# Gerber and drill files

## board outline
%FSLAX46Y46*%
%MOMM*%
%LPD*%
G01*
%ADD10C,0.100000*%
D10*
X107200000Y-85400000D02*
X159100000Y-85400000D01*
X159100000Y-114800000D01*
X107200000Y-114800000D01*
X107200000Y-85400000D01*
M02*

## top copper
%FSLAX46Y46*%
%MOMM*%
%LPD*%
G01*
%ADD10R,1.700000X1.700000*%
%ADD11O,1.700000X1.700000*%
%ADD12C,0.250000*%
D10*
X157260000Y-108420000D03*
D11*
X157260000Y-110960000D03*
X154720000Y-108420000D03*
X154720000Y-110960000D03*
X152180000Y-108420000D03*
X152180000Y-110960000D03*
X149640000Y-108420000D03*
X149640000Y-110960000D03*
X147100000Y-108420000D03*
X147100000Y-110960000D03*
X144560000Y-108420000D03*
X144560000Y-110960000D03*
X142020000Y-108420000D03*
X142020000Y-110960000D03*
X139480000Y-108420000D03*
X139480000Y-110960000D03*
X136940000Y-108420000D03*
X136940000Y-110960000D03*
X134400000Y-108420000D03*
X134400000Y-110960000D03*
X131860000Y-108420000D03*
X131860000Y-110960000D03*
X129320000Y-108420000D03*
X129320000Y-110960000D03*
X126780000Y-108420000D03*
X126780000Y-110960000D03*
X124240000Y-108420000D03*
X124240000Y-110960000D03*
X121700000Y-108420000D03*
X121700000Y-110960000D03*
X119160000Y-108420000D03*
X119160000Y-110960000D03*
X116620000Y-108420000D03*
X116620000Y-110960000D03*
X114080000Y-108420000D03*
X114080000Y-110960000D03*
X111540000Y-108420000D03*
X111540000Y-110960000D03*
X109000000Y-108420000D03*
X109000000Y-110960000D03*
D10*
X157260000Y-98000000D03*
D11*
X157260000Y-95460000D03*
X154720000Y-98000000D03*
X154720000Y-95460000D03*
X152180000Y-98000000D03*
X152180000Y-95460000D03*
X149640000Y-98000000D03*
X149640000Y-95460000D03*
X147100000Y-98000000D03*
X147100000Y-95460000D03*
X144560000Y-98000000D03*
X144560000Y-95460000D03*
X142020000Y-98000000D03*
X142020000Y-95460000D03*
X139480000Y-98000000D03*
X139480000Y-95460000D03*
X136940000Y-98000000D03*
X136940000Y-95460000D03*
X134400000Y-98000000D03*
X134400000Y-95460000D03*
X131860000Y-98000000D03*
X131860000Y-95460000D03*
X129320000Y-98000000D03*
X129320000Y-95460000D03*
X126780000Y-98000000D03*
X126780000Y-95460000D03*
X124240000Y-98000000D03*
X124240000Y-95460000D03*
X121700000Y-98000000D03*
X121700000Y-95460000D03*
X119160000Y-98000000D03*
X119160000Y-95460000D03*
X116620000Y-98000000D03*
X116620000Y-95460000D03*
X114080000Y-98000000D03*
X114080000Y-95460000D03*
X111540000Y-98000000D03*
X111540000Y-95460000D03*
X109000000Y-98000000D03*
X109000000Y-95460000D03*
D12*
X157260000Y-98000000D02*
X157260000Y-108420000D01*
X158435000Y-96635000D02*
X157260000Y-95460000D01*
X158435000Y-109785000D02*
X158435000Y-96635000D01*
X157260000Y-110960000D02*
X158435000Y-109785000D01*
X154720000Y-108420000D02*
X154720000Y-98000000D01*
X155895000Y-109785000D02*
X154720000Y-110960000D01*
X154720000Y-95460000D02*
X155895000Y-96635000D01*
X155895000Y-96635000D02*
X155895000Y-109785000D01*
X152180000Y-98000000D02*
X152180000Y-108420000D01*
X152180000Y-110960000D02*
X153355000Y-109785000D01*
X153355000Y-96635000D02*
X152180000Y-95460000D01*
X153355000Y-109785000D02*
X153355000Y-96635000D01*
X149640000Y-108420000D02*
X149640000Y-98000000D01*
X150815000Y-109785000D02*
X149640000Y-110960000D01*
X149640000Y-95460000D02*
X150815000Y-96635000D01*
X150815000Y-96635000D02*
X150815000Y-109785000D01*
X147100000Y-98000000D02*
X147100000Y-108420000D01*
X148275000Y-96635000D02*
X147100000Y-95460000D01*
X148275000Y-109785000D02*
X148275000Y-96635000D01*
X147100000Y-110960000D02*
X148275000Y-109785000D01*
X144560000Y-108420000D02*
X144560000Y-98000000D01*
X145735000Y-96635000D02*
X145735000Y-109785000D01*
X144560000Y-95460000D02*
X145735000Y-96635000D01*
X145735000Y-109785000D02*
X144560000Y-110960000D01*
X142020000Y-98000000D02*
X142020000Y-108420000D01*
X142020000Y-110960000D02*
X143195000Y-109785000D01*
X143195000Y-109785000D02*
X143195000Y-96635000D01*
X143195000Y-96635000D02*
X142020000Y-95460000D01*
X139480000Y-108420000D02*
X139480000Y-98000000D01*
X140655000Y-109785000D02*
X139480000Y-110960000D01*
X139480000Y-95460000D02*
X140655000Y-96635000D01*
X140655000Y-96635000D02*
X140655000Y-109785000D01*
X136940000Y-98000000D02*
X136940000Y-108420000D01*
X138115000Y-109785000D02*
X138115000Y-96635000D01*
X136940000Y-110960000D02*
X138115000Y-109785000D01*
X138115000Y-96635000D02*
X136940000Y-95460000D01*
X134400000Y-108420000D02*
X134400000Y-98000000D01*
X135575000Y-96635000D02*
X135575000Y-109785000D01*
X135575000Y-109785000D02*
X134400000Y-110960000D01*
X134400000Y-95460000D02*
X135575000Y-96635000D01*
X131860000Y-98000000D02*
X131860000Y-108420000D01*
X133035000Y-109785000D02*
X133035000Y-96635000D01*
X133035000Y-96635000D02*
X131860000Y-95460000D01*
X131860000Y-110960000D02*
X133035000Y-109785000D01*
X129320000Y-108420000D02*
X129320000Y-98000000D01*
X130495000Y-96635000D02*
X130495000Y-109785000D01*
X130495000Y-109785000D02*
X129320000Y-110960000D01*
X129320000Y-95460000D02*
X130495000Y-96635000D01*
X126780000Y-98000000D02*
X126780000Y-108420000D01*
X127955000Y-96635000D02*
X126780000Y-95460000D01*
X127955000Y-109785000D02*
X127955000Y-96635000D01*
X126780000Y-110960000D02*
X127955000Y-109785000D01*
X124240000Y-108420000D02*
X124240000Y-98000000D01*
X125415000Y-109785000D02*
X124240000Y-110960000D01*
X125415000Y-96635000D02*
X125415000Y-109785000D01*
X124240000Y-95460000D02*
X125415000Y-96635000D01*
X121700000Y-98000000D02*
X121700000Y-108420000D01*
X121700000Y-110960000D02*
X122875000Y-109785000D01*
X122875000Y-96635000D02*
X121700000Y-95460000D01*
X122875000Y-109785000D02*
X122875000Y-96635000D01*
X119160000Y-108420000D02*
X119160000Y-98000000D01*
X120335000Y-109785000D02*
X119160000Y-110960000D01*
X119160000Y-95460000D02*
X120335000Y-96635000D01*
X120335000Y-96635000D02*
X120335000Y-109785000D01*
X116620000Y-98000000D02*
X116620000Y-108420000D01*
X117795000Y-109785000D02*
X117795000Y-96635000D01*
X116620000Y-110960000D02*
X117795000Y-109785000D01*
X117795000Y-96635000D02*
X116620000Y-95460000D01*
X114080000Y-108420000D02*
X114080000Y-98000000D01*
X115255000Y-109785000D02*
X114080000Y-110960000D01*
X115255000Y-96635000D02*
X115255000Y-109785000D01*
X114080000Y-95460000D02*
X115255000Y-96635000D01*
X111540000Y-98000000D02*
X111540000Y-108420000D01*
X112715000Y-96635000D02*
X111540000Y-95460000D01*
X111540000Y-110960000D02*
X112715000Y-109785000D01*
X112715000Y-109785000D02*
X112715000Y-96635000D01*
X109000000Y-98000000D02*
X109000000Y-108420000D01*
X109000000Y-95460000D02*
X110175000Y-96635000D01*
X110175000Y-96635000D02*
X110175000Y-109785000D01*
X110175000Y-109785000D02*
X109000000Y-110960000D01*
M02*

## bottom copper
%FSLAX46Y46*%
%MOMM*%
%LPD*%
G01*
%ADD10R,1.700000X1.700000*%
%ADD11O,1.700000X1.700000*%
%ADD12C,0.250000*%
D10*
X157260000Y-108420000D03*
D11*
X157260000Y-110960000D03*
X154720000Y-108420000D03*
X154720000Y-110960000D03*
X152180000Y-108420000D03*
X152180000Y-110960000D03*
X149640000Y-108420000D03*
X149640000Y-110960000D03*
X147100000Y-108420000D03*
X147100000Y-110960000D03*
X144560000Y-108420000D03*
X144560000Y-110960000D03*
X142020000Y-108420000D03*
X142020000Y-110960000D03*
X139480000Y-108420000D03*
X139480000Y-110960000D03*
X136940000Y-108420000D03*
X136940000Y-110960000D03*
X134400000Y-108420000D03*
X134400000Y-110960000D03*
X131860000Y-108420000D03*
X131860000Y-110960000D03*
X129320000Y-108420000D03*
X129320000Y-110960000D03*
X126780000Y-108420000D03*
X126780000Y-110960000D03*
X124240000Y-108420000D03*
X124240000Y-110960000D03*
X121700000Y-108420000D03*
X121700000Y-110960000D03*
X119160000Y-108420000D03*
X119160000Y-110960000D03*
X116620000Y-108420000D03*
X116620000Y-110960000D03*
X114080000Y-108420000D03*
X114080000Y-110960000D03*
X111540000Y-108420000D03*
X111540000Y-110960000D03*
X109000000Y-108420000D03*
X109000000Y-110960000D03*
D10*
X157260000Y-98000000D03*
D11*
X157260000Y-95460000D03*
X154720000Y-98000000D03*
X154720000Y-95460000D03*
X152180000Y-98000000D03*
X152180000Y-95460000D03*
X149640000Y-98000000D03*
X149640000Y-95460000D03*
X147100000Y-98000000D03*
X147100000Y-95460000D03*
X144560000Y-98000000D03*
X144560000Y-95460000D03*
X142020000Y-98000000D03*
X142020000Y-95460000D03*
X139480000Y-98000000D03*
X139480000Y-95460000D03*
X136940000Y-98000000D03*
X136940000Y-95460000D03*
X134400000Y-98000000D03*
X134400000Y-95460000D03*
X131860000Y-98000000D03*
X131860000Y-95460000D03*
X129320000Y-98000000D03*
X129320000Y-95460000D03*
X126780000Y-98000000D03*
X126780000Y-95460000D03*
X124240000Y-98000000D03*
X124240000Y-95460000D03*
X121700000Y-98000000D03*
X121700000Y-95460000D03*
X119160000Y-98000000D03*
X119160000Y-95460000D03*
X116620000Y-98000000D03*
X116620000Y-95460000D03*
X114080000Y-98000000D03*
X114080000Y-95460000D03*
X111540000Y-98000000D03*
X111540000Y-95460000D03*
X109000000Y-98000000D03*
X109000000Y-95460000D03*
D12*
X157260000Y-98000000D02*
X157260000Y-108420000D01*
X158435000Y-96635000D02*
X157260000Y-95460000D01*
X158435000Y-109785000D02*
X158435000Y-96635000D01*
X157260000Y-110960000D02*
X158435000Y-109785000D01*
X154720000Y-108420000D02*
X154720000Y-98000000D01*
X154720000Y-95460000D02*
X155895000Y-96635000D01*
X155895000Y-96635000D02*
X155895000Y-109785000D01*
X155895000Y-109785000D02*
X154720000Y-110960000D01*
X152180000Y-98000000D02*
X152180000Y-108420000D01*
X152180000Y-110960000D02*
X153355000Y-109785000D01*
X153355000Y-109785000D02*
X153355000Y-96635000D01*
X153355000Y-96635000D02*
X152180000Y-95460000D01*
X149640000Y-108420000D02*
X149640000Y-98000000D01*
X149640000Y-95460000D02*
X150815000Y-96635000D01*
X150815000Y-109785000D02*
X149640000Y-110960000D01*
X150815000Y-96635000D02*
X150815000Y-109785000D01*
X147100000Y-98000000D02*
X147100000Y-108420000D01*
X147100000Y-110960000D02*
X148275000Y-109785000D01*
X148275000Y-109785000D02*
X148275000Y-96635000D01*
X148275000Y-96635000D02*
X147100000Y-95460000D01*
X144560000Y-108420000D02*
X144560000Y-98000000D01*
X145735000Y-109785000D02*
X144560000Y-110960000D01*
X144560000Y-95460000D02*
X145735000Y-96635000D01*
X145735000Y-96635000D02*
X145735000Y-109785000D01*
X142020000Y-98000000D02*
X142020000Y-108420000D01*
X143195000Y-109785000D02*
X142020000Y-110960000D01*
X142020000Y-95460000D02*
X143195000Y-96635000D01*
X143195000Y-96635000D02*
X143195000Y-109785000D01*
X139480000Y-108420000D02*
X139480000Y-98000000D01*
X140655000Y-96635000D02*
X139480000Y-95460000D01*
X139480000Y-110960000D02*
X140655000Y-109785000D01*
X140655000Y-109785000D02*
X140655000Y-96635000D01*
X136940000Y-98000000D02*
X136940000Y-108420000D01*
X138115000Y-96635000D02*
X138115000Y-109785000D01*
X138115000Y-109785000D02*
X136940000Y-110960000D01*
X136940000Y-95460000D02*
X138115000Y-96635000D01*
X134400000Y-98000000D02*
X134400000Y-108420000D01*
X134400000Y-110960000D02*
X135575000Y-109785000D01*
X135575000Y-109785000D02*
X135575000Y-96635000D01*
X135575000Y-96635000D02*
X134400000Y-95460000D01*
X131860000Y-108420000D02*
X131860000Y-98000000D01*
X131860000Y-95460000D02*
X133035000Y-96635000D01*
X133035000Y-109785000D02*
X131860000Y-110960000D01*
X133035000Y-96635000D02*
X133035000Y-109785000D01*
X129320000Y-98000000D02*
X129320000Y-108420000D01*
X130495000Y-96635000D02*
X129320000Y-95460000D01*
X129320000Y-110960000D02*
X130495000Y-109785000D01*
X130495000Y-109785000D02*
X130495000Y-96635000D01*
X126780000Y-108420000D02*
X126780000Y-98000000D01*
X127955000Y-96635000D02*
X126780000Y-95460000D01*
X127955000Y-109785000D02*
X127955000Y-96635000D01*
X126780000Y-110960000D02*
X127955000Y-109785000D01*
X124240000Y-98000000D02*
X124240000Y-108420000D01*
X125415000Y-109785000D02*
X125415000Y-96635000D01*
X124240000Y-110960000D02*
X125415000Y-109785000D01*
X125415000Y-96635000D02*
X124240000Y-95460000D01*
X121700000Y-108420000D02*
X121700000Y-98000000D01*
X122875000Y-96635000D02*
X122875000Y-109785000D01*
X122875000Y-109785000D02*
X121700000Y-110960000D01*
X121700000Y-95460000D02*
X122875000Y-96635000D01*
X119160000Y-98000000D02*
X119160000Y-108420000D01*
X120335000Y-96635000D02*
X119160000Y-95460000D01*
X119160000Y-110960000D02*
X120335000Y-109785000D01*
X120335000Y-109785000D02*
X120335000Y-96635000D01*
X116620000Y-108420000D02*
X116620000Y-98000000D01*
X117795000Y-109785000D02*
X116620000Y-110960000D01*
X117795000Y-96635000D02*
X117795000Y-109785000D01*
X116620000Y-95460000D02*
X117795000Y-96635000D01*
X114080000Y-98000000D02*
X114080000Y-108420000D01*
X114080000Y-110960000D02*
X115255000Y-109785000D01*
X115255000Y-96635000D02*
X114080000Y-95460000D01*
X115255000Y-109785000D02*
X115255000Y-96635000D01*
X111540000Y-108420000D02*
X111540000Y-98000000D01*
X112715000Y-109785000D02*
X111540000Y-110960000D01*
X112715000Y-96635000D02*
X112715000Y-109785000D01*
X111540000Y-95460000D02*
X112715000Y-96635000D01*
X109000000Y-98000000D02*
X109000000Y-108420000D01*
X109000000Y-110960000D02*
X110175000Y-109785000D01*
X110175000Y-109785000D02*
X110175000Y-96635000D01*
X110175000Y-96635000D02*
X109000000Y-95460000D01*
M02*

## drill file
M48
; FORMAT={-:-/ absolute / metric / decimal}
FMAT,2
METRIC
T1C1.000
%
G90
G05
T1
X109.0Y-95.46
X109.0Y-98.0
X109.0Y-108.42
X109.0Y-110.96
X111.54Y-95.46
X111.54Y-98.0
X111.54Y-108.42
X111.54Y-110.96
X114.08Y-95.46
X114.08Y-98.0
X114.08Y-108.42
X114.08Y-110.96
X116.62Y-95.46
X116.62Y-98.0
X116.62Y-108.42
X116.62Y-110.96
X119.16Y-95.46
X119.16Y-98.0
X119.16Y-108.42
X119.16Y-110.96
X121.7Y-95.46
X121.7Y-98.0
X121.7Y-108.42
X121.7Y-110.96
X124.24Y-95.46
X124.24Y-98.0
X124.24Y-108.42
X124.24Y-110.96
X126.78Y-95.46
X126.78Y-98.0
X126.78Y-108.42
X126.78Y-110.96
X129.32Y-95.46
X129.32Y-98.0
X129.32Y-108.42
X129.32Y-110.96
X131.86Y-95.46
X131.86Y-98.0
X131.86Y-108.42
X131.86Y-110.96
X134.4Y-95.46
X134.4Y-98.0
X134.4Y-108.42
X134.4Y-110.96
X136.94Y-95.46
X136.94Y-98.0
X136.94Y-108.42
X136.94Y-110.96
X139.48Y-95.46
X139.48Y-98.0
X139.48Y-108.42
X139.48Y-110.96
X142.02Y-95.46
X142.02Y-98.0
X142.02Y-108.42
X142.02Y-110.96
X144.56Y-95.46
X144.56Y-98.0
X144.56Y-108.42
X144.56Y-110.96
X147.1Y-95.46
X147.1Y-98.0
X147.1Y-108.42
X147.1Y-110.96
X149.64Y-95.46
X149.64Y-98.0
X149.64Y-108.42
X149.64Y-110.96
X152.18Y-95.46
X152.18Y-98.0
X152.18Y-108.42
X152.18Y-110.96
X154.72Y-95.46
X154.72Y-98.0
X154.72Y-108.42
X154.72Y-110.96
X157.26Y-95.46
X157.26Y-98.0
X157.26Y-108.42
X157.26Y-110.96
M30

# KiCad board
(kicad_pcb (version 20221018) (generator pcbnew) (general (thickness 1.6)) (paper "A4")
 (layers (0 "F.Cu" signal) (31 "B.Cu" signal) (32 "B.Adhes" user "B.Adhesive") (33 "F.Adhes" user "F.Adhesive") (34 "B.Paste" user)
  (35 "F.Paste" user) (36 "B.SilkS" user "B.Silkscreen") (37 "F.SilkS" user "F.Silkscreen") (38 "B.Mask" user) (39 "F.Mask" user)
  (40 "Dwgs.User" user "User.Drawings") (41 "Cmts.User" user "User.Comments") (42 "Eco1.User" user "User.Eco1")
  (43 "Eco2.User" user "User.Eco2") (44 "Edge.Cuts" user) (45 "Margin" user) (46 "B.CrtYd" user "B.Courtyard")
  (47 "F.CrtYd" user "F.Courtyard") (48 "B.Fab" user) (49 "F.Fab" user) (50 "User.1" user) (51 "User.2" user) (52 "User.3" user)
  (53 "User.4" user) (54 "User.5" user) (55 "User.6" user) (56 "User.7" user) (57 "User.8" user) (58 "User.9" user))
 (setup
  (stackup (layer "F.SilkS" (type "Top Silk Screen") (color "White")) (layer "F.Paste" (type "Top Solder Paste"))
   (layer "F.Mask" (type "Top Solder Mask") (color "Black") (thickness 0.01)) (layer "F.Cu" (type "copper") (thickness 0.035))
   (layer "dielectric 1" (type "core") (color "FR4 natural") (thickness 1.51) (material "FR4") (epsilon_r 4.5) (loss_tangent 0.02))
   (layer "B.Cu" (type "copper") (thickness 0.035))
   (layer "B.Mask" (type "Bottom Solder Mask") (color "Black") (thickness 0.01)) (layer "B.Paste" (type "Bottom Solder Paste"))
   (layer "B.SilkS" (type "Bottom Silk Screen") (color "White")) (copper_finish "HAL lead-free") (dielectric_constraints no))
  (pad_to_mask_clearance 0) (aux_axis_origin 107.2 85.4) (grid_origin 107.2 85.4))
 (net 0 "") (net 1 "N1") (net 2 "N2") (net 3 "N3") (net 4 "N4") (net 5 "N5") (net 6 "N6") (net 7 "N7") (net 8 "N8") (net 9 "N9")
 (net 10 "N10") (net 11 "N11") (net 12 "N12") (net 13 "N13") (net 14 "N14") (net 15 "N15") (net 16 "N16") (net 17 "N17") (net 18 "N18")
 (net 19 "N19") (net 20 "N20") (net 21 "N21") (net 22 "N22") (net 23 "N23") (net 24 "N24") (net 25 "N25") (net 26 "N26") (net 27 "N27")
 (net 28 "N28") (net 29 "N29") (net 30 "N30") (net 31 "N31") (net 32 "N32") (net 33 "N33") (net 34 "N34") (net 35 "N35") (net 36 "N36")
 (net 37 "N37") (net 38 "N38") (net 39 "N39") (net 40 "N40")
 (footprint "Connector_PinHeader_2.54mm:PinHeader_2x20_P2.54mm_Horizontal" (layer "F.Cu") (at 157.26 108.42 -90)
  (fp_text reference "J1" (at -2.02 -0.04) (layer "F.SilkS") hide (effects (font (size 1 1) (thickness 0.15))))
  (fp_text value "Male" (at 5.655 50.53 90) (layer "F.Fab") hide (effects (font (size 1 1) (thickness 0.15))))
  (pad "1" thru_hole rect (at 0 0 270) (size 1.7 1.7) (drill 1) (layers "*.Cu" "*.Mask") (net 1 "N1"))
  (pad "2" thru_hole oval (at 2.54 0 270) (size 1.7 1.7) (drill 1) (layers "*.Cu" "*.Mask") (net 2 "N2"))
  (pad "3" thru_hole oval (at 0 2.54 270) (size 1.7 1.7) (drill 1) (layers "*.Cu" "*.Mask") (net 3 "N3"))
  (pad "4" thru_hole oval (at 2.54 2.54 270) (size 1.7 1.7) (drill 1) (layers "*.Cu" "*.Mask") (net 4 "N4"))
  (pad "5" thru_hole oval (at 0 5.08 270) (size 1.7 1.7) (drill 1) (layers "*.Cu" "*.Mask") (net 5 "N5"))
  (pad "6" thru_hole oval (at 2.54 5.08 270) (size 1.7 1.7) (drill 1) (layers "*.Cu" "*.Mask") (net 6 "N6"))
  (pad "7" thru_hole oval (at 0 7.62 270) (size 1.7 1.7) (drill 1) (layers "*.Cu" "*.Mask") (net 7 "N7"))
  (pad "8" thru_hole oval (at 2.54 7.62 270) (size 1.7 1.7) (drill 1) (layers "*.Cu" "*.Mask") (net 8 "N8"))
  (pad "9" thru_hole oval (at 0 10.16 270) (size 1.7 1.7) (drill 1) (layers "*.Cu" "*.Mask") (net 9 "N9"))
  (pad "10" thru_hole oval (at 2.54 10.16 270) (size 1.7 1.7) (drill 1) (layers "*.Cu" "*.Mask") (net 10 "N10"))
  (pad "11" thru_hole oval (at 0 12.7 270) (size 1.7 1.7) (drill 1) (layers "*.Cu" "*.Mask") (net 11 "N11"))
  (pad "12" thru_hole oval (at 2.54 12.7 270) (size 1.7 1.7) (drill 1) (layers "*.Cu" "*.Mask") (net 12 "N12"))
  (pad "13" thru_hole oval (at 0 15.24 270) (size 1.7 1.7) (drill 1) (layers "*.Cu" "*.Mask") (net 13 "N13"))
  (pad "14" thru_hole oval (at 2.54 15.24 270) (size 1.7 1.7) (drill 1) (layers "*.Cu" "*.Mask") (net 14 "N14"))
  (pad "15" thru_hole oval (at 0 17.78 270) (size 1.7 1.7) (drill 1) (layers "*.Cu" "*.Mask") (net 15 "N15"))
  (pad "16" thru_hole oval (at 2.54 17.78 270) (size 1.7 1.7) (drill 1) (layers "*.Cu" "*.Mask") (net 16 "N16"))
  (pad "17" thru_hole oval (at 0 20.32 270) (size 1.7 1.7) (drill 1) (layers "*.Cu" "*.Mask") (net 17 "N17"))
  (pad "18" thru_hole oval (at 2.54 20.32 270) (size 1.7 1.7) (drill 1) (layers "*.Cu" "*.Mask") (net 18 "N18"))
  (pad "19" thru_hole oval (at 0 22.86 270) (size 1.7 1.7) (drill 1) (layers "*.Cu" "*.Mask") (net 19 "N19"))
  (pad "20" thru_hole oval (at 2.54 22.86 270) (size 1.7 1.7) (drill 1) (layers "*.Cu" "*.Mask") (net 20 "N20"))
  (pad "21" thru_hole oval (at 0 25.4 270) (size 1.7 1.7) (drill 1) (layers "*.Cu" "*.Mask") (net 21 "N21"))
  (pad "22" thru_hole oval (at 2.54 25.4 270) (size 1.7 1.7) (drill 1) (layers "*.Cu" "*.Mask") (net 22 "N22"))
  (pad "23" thru_hole oval (at 0 27.94 270) (size 1.7 1.7) (drill 1) (layers "*.Cu" "*.Mask") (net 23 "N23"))
  (pad "24" thru_hole oval (at 2.54 27.94 270) (size 1.7 1.7) (drill 1) (layers "*.Cu" "*.Mask") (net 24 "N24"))
  (pad "25" thru_hole oval (at 0 30.48 270) (size 1.7 1.7) (drill 1) (layers "*.Cu" "*.Mask") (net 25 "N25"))
  (pad "26" thru_hole oval (at 2.54 30.48 270) (size 1.7 1.7) (drill 1) (layers "*.Cu" "*.Mask") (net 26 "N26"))
  (pad "27" thru_hole oval (at 0 33.02 270) (size 1.7 1.7) (drill 1) (layers "*.Cu" "*.Mask") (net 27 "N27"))
  (pad "28" thru_hole oval (at 2.54 33.02 270) (size 1.7 1.7) (drill 1) (layers "*.Cu" "*.Mask") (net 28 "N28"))
  (pad "29" thru_hole oval (at 0 35.56 270) (size 1.7 1.7) (drill 1) (layers "*.Cu" "*.Mask") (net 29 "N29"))
  (pad "30" thru_hole oval (at 2.54 35.56 270) (size 1.7 1.7) (drill 1) (layers "*.Cu" "*.Mask") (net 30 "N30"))
  (pad "31" thru_hole oval (at 0 38.1 270) (size 1.7 1.7) (drill 1) (layers "*.Cu" "*.Mask") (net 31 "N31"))
  (pad "32" thru_hole oval (at 2.54 38.1 270) (size 1.7 1.7) (drill 1) (layers "*.Cu" "*.Mask") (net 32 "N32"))
  (pad "33" thru_hole oval (at 0 40.64 270) (size 1.7 1.7) (drill 1) (layers "*.Cu" "*.Mask") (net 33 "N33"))
  (pad "34" thru_hole oval (at 2.54 40.64 270) (size 1.7 1.7) (drill 1) (layers "*.Cu" "*.Mask") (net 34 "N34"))
  (pad "35" thru_hole oval (at 0 43.18 270) (size 1.7 1.7) (drill 1) (layers "*.Cu" "*.Mask") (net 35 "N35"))
  (pad "36" thru_hole oval (at 2.54 43.18 270) (size 1.7 1.7) (drill 1) (layers "*.Cu" "*.Mask") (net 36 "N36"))
  (pad "37" thru_hole oval (at 0 45.72 270) (size 1.7 1.7) (drill 1) (layers "*.Cu" "*.Mask") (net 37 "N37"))
  (pad "38" thru_hole oval (at 2.54 45.72 270) (size 1.7 1.7) (drill 1) (layers "*.Cu" "*.Mask") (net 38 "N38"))
  (pad "39" thru_hole oval (at 0 48.26 270) (size 1.7 1.7) (drill 1) (layers "*.Cu" "*.Mask") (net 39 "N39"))
  (pad "40" thru_hole oval (at 2.54 48.26 270) (size 1.7 1.7) (drill 1) (layers "*.Cu" "*.Mask") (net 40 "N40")))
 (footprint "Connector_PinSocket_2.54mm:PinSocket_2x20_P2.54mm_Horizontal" (layer "F.Cu") (at 157.26 98 -90)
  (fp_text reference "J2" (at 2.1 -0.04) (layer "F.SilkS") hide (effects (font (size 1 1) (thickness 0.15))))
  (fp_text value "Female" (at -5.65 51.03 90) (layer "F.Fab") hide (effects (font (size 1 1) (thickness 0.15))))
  (pad "1" thru_hole rect (at 0 0 270) (size 1.7 1.7) (drill 1) (layers "*.Cu" "*.Mask") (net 1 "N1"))
  (pad "2" thru_hole oval (at -2.54 0 270) (size 1.7 1.7) (drill 1) (layers "*.Cu" "*.Mask") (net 2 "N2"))
  (pad "3" thru_hole oval (at 0 2.54 270) (size 1.7 1.7) (drill 1) (layers "*.Cu" "*.Mask") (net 3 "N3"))
  (pad "4" thru_hole oval (at -2.54 2.54 270) (size 1.7 1.7) (drill 1) (layers "*.Cu" "*.Mask") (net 4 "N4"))
  (pad "5" thru_hole oval (at 0 5.08 270) (size 1.7 1.7) (drill 1) (layers "*.Cu" "*.Mask") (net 5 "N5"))
  (pad "6" thru_hole oval (at -2.54 5.08 270) (size 1.7 1.7) (drill 1) (layers "*.Cu" "*.Mask") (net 6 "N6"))
  (pad "7" thru_hole oval (at 0 7.62 270) (size 1.7 1.7) (drill 1) (layers "*.Cu" "*.Mask") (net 7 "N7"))
  (pad "8" thru_hole oval (at -2.54 7.62 270) (size 1.7 1.7) (drill 1) (layers "*.Cu" "*.Mask") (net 8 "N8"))
  (pad "9" thru_hole oval (at 0 10.16 270) (size 1.7 1.7) (drill 1) (layers "*.Cu" "*.Mask") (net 9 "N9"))
  (pad "10" thru_hole oval (at -2.54 10.16 270) (size 1.7 1.7) (drill 1) (layers "*.Cu" "*.Mask") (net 10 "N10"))
  (pad "11" thru_hole oval (at 0 12.7 270) (size 1.7 1.7) (drill 1) (layers "*.Cu" "*.Mask") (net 11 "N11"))
  (pad "12" thru_hole oval (at -2.54 12.7 270) (size 1.7 1.7) (drill 1) (layers "*.Cu" "*.Mask") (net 12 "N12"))
  (pad "13" thru_hole oval (at 0 15.24 270) (size 1.7 1.7) (drill 1) (layers "*.Cu" "*.Mask") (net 13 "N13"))
  (pad "14" thru_hole oval (at -2.54 15.24 270) (size 1.7 1.7) (drill 1) (layers "*.Cu" "*.Mask") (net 14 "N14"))
  (pad "15" thru_hole oval (at 0 17.78 270) (size 1.7 1.7) (drill 1) (layers "*.Cu" "*.Mask") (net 15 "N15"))
  (pad "16" thru_hole oval (at -2.54 17.78 270) (size 1.7 1.7) (drill 1) (layers "*.Cu" "*.Mask") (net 16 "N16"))
  (pad "17" thru_hole oval (at 0 20.32 270) (size 1.7 1.7) (drill 1) (layers "*.Cu" "*.Mask") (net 17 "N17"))
  (pad "18" thru_hole oval (at -2.54 20.32 270) (size 1.7 1.7) (drill 1) (layers "*.Cu" "*.Mask") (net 18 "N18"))
  (pad "19" thru_hole oval (at 0 22.86 270) (size 1.7 1.7) (drill 1) (layers "*.Cu" "*.Mask") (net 19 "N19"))
  (pad "20" thru_hole oval (at -2.54 22.86 270) (size 1.7 1.7) (drill 1) (layers "*.Cu" "*.Mask") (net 20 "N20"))
  (pad "21" thru_hole oval (at 0 25.4 270) (size 1.7 1.7) (drill 1) (layers "*.Cu" "*.Mask") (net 21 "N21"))
  (pad "22" thru_hole oval (at -2.54 25.4 270) (size 1.7 1.7) (drill 1) (layers "*.Cu" "*.Mask") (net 22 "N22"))
  (pad "23" thru_hole oval (at 0 27.94 270) (size 1.7 1.7) (drill 1) (layers "*.Cu" "*.Mask") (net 23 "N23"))
  (pad "24" thru_hole oval (at -2.54 27.94 270) (size 1.7 1.7) (drill 1) (layers "*.Cu" "*.Mask") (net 24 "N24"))
  (pad "25" thru_hole oval (at 0 30.48 270) (size 1.7 1.7) (drill 1) (layers "*.Cu" "*.Mask") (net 25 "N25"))
  (pad "26" thru_hole oval (at -2.54 30.48 270) (size 1.7 1.7) (drill 1) (layers "*.Cu" "*.Mask") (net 26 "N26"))
  (pad "27" thru_hole oval (at 0 33.02 270) (size 1.7 1.7) (drill 1) (layers "*.Cu" "*.Mask") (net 27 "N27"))
  (pad "28" thru_hole oval (at -2.54 33.02 270) (size 1.7 1.7) (drill 1) (layers "*.Cu" "*.Mask") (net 28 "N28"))
  (pad "29" thru_hole oval (at 0 35.56 270) (size 1.7 1.7) (drill 1) (layers "*.Cu" "*.Mask") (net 29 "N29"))
  (pad "30" thru_hole oval (at -2.54 35.56 270) (size 1.7 1.7) (drill 1) (layers "*.Cu" "*.Mask") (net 30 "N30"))
  (pad "31" thru_hole oval (at 0 38.1 270) (size 1.7 1.7) (drill 1) (layers "*.Cu" "*.Mask") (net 31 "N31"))
  (pad "32" thru_hole oval (at -2.54 38.1 270) (size 1.7 1.7) (drill 1) (layers "*.Cu" "*.Mask") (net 32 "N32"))
  (pad "33" thru_hole oval (at 0 40.64 270) (size 1.7 1.7) (drill 1) (layers "*.Cu" "*.Mask") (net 33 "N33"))
  (pad "34" thru_hole oval (at -2.54 40.64 270) (size 1.7 1.7) (drill 1) (layers "*.Cu" "*.Mask") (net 34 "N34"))
  (pad "35" thru_hole oval (at 0 43.18 270) (size 1.7 1.7) (drill 1) (layers "*.Cu" "*.Mask") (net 35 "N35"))
  (pad "36" thru_hole oval (at -2.54 43.18 270) (size 1.7 1.7) (drill 1) (layers "*.Cu" "*.Mask") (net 36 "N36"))
  (pad "37" thru_hole oval (at 0 45.72 270) (size 1.7 1.7) (drill 1) (layers "*.Cu" "*.Mask") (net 37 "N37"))
  (pad "38" thru_hole oval (at -2.54 45.72 270) (size 1.7 1.7) (drill 1) (layers "*.Cu" "*.Mask") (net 38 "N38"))
  (pad "39" thru_hole oval (at 0 48.26 270) (size 1.7 1.7) (drill 1) (layers "*.Cu" "*.Mask") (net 39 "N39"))
  (pad "40" thru_hole oval (at -2.54 48.26 270) (size 1.7 1.7) (drill 1) (layers "*.Cu" "*.Mask") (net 40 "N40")))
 (gr_rect (start 107.2 85.4) (end 159.1 114.8) (stroke (width 0.1) (type default)) (fill none) (layer "Edge.Cuts"))
 (segment (start 157.26 98) (end 157.26 108.42) (width 0.25) (layer "F.Cu") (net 1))
 (segment (start 157.26 98) (end 157.26 108.42) (width 0.25) (layer "B.Cu") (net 1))
 (segment (start 158.435 96.635) (end 157.26 95.46) (width 0.25) (layer "F.Cu") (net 2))
 (segment (start 158.435 109.785) (end 158.435 96.635) (width 0.25) (layer "F.Cu") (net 2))
 (segment (start 157.26 110.96) (end 158.435 109.785) (width 0.25) (layer "F.Cu") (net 2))
 (segment (start 158.435 96.635) (end 157.26 95.46) (width 0.25) (layer "B.Cu") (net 2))
 (segment (start 158.435 109.785) (end 158.435 96.635) (width 0.25) (layer "B.Cu") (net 2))
 (segment (start 157.26 110.96) (end 158.435 109.785) (width 0.25) (layer "B.Cu") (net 2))
 (segment (start 154.72 108.42) (end 154.72 98) (width 0.25) (layer "F.Cu") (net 3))
 (segment (start 154.72 108.42) (end 154.72 98) (width 0.25) (layer "B.Cu") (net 3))
 (segment (start 155.895 109.785) (end 154.72 110.96) (width 0.25) (layer "F.Cu") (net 4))
 (segment (start 154.72 95.46) (end 155.895 96.635) (width 0.25) (layer "F.Cu") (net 4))
 (segment (start 155.895 96.635) (end 155.895 109.785) (width 0.25) (layer "F.Cu") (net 4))
 (segment (start 154.72 95.46) (end 155.895 96.635) (width 0.25) (layer "B.Cu") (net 4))
 (segment (start 155.895 96.635) (end 155.895 109.785) (width 0.25) (layer "B.Cu") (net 4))
 (segment (start 155.895 109.785) (end 154.72 110.96) (width 0.25) (layer "B.Cu") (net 4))
 (segment (start 152.18 98) (end 152.18 108.42) (width 0.25) (layer "F.Cu") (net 5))
 (segment (start 152.18 98) (end 152.18 108.42) (width 0.25) (layer "B.Cu") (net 5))
 (segment (start 152.18 110.96) (end 153.355 109.785) (width 0.25) (layer "F.Cu") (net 6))
 (segment (start 153.355 96.635) (end 152.18 95.46) (width 0.25) (layer "F.Cu") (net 6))
 (segment (start 153.355 109.785) (end 153.355 96.635) (width 0.25) (layer "F.Cu") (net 6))
 (segment (start 152.18 110.96) (end 153.355 109.785) (width 0.25) (layer "B.Cu") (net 6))
 (segment (start 153.355 109.785) (end 153.355 96.635) (width 0.25) (layer "B.Cu") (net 6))
 (segment (start 153.355 96.635) (end 152.18 95.46) (width 0.25) (layer "B.Cu") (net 6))
 (segment (start 149.64 108.42) (end 149.64 98) (width 0.25) (layer "F.Cu") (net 7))
 (segment (start 149.64 108.42) (end 149.64 98) (width 0.25) (layer "B.Cu") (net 7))
 (segment (start 150.815 109.785) (end 149.64 110.96) (width 0.25) (layer "F.Cu") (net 8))
 (segment (start 149.64 95.46) (end 150.815 96.635) (width 0.25) (layer "F.Cu") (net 8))
 (segment (start 150.815 96.635) (end 150.815 109.785) (width 0.25) (layer "F.Cu") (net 8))
 (segment (start 149.64 95.46) (end 150.815 96.635) (width 0.25) (layer "B.Cu") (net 8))
 (segment (start 150.815 109.785) (end 149.64 110.96) (width 0.25) (layer "B.Cu") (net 8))
 (segment (start 150.815 96.635) (end 150.815 109.785) (width 0.25) (layer "B.Cu") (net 8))
 (segment (start 147.1 98) (end 147.1 108.42) (width 0.25) (layer "F.Cu") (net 9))
 (segment (start 147.1 98) (end 147.1 108.42) (width 0.25) (layer "B.Cu") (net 9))
 (segment (start 148.275 96.635) (end 147.1 95.46) (width 0.25) (layer "F.Cu") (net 10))
 (segment (start 148.275 109.785) (end 148.275 96.635) (width 0.25) (layer "F.Cu") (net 10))
 (segment (start 147.1 110.96) (end 148.275 109.785) (width 0.25) (layer "F.Cu") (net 10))
 (segment (start 147.1 110.96) (end 148.275 109.785) (width 0.25) (layer "B.Cu") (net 10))
 (segment (start 148.275 109.785) (end 148.275 96.635) (width 0.25) (layer "B.Cu") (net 10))
 (segment (start 148.275 96.635) (end 147.1 95.46) (width 0.25) (layer "B.Cu") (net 10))
 (segment (start 144.56 108.42) (end 144.56 98) (width 0.25) (layer "F.Cu") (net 11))
 (segment (start 144.56 108.42) (end 144.56 98) (width 0.25) (layer "B.Cu") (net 11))
 (segment (start 145.735 96.635) (end 145.735 109.785) (width 0.25) (layer "F.Cu") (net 12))
 (segment (start 144.56 95.46) (end 145.735 96.635) (width 0.25) (layer "F.Cu") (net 12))
 (segment (start 145.735 109.785) (end 144.56 110.96) (width 0.25) (layer "F.Cu") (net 12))
 (segment (start 145.735 109.785) (end 144.56 110.96) (width 0.25) (layer "B.Cu") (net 12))
 (segment (start 144.56 95.46) (end 145.735 96.635) (width 0.25) (layer "B.Cu") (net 12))
 (segment (start 145.735 96.635) (end 145.735 109.785) (width 0.25) (layer "B.Cu") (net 12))
 (segment (start 142.02 98) (end 142.02 108.42) (width 0.25) (layer "F.Cu") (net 13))
 (segment (start 142.02 98) (end 142.02 108.42) (width 0.25) (layer "B.Cu") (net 13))
 (segment (start 142.02 110.96) (end 143.195 109.785) (width 0.25) (layer "F.Cu") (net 14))
 (segment (start 143.195 109.785) (end 143.195 96.635) (width 0.25) (layer "F.Cu") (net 14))
 (segment (start 143.195 96.635) (end 142.02 95.46) (width 0.25) (layer "F.Cu") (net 14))
 (segment (start 143.195 109.785) (end 142.02 110.96) (width 0.25) (layer "B.Cu") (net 14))
 (segment (start 142.02 95.46) (end 143.195 96.635) (width 0.25) (layer "B.Cu") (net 14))
 (segment (start 143.195 96.635) (end 143.195 109.785) (width 0.25) (layer "B.Cu") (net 14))
 (segment (start 139.48 108.42) (end 139.48 98) (width 0.25) (layer "F.Cu") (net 15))
 (segment (start 139.48 108.42) (end 139.48 98) (width 0.25) (layer "B.Cu") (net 15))
 (segment (start 140.655 109.785) (end 139.48 110.96) (width 0.25) (layer "F.Cu") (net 16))
 (segment (start 139.48 95.46) (end 140.655 96.635) (width 0.25) (layer "F.Cu") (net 16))
 (segment (start 140.655 96.635) (end 140.655 109.785) (width 0.25) (layer "F.Cu") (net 16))
 (segment (start 140.655 96.635) (end 139.48 95.46) (width 0.25) (layer "B.Cu") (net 16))
 (segment (start 139.48 110.96) (end 140.655 109.785) (width 0.25) (layer "B.Cu") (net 16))
 (segment (start 140.655 109.785) (end 140.655 96.635) (width 0.25) (layer "B.Cu") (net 16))
 (segment (start 136.94 98) (end 136.94 108.42) (width 0.25) (layer "F.Cu") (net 17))
 (segment (start 136.94 98) (end 136.94 108.42) (width 0.25) (layer "B.Cu") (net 17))
 (segment (start 138.115 109.785) (end 138.115 96.635) (width 0.25) (layer "F.Cu") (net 18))
 (segment (start 136.94 110.96) (end 138.115 109.785) (width 0.25) (layer "F.Cu") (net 18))
 (segment (start 138.115 96.635) (end 136.94 95.46) (width 0.25) (layer "F.Cu") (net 18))
 (segment (start 138.115 96.635) (end 138.115 109.785) (width 0.25) (layer "B.Cu") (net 18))
 (segment (start 138.115 109.785) (end 136.94 110.96) (width 0.25) (layer "B.Cu") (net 18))
 (segment (start 136.94 95.46) (end 138.115 96.635) (width 0.25) (layer "B.Cu") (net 18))
 (segment (start 134.4 108.42) (end 134.4 98) (width 0.25) (layer "F.Cu") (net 19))
 (segment (start 134.4 98) (end 134.4 108.42) (width 0.25) (layer "B.Cu") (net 19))
 (segment (start 135.575 96.635) (end 135.575 109.785) (width 0.25) (layer "F.Cu") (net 20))
 (segment (start 135.575 109.785) (end 134.4 110.96) (width 0.25) (layer "F.Cu") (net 20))
 (segment (start 134.4 95.46) (end 135.575 96.635) (width 0.25) (layer "F.Cu") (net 20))
 (segment (start 134.4 110.96) (end 135.575 109.785) (width 0.25) (layer "B.Cu") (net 20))
 (segment (start 135.575 109.785) (end 135.575 96.635) (width 0.25) (layer "B.Cu") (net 20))
 (segment (start 135.575 96.635) (end 134.4 95.46) (width 0.25) (layer "B.Cu") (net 20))
 (segment (start 131.86 98) (end 131.86 108.42) (width 0.25) (layer "F.Cu") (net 21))
 (segment (start 131.86 108.42) (end 131.86 98) (width 0.25) (layer "B.Cu") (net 21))
 (segment (start 133.035 109.785) (end 133.035 96.635) (width 0.25) (layer "F.Cu") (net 22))
 (segment (start 133.035 96.635) (end 131.86 95.46) (width 0.25) (layer "F.Cu") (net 22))
 (segment (start 131.86 110.96) (end 133.035 109.785) (width 0.25) (layer "F.Cu") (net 22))
 (segment (start 131.86 95.46) (end 133.035 96.635) (width 0.25) (layer "B.Cu") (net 22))
 (segment (start 133.035 109.785) (end 131.86 110.96) (width 0.25) (layer "B.Cu") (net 22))
 (segment (start 133.035 96.635) (end 133.035 109.785) (width 0.25) (layer "B.Cu") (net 22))
 (segment (start 129.32 108.42) (end 129.32 98) (width 0.25) (layer "F.Cu") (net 23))
 (segment (start 129.32 98) (end 129.32 108.42) (width 0.25) (layer "B.Cu") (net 23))
 (segment (start 130.495 96.635) (end 130.495 109.785) (width 0.25) (layer "F.Cu") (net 24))
 (segment (start 130.495 109.785) (end 129.32 110.96) (width 0.25) (layer "F.Cu") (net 24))
 (segment (start 129.32 95.46) (end 130.495 96.635) (width 0.25) (layer "F.Cu") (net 24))
 (segment (start 130.495 96.635) (end 129.32 95.46) (width 0.25) (layer "B.Cu") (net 24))
 (segment (start 129.32 110.96) (end 130.495 109.785) (width 0.25) (layer "B.Cu") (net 24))
 (segment (start 130.495 109.785) (end 130.495 96.635) (width 0.25) (layer "B.Cu") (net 24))
 (segment (start 126.78 98) (end 126.78 108.42) (width 0.25) (layer "F.Cu") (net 25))
 (segment (start 126.78 108.42) (end 126.78 98) (width 0.25) (layer "B.Cu") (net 25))
 (segment (start 127.955 96.635) (end 126.78 95.46) (width 0.25) (layer "F.Cu") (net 26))
 (segment (start 127.955 109.785) (end 127.955 96.635) (width 0.25) (layer "F.Cu") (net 26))
 (segment (start 126.78 110.96) (end 127.955 109.785) (width 0.25) (layer "F.Cu") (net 26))
 (segment (start 127.955 96.635) (end 126.78 95.46) (width 0.25) (layer "B.Cu") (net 26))
 (segment (start 127.955 109.785) (end 127.955 96.635) (width 0.25) (layer "B.Cu") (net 26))
 (segment (start 126.78 110.96) (end 127.955 109.785) (width 0.25) (layer "B.Cu") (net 26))
 (segment (start 124.24 108.42) (end 124.24 98) (width 0.25) (layer "F.Cu") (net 27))
 (segment (start 124.24 98) (end 124.24 108.42) (width 0.25) (layer "B.Cu") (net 27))
 (segment (start 125.415 109.785) (end 124.24 110.96) (width 0.25) (layer "F.Cu") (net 28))
 (segment (start 125.415 96.635) (end 125.415 109.785) (width 0.25) (layer "F.Cu") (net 28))
 (segment (start 124.24 95.46) (end 125.415 96.635) (width 0.25) (layer "F.Cu") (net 28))
 (segment (start 125.415 109.785) (end 125.415 96.635) (width 0.25) (layer "B.Cu") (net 28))
 (segment (start 124.24 110.96) (end 125.415 109.785) (width 0.25) (layer "B.Cu") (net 28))
 (segment (start 125.415 96.635) (end 124.24 95.46) (width 0.25) (layer "B.Cu") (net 28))
 (segment (start 121.7 98) (end 121.7 108.42) (width 0.25) (layer "F.Cu") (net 29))
 (segment (start 121.7 108.42) (end 121.7 98) (width 0.25) (layer "B.Cu") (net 29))
 (segment (start 121.7 110.96) (end 122.875 109.785) (width 0.25) (layer "F.Cu") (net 30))
 (segment (start 122.875 96.635) (end 121.7 95.46) (width 0.25) (layer "F.Cu") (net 30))
 (segment (start 122.875 109.785) (end 122.875 96.635) (width 0.25) (layer "F.Cu") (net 30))
 (segment (start 122.875 96.635) (end 122.875 109.785) (width 0.25) (layer "B.Cu") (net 30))
 (segment (start 122.875 109.785) (end 121.7 110.96) (width 0.25) (layer "B.Cu") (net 30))
 (segment (start 121.7 95.46) (end 122.875 96.635) (width 0.25) (layer "B.Cu") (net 30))
 (segment (start 119.16 108.42) (end 119.16 98) (width 0.25) (layer "F.Cu") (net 31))
 (segment (start 119.16 98) (end 119.16 108.42) (width 0.25) (layer "B.Cu") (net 31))
 (segment (start 120.335 109.785) (end 119.16 110.96) (width 0.25) (layer "F.Cu") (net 32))
 (segment (start 119.16 95.46) (end 120.335 96.635) (width 0.25) (layer "F.Cu") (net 32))
 (segment (start 120.335 96.635) (end 120.335 109.785) (width 0.25) (layer "F.Cu") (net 32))
 (segment (start 120.335 96.635) (end 119.16 95.46) (width 0.25) (layer "B.Cu") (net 32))
 (segment (start 119.16 110.96) (end 120.335 109.785) (width 0.25) (layer "B.Cu") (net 32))
 (segment (start 120.335 109.785) (end 120.335 96.635) (width 0.25) (layer "B.Cu") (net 32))
 (segment (start 116.62 98) (end 116.62 108.42) (width 0.25) (layer "F.Cu") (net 33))
 (segment (start 116.62 108.42) (end 116.62 98) (width 0.25) (layer "B.Cu") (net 33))
 (segment (start 117.795 109.785) (end 117.795 96.635) (width 0.25) (layer "F.Cu") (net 34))
 (segment (start 116.62 110.96) (end 117.795 109.785) (width 0.25) (layer "F.Cu") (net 34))
 (segment (start 117.795 96.635) (end 116.62 95.46) (width 0.25) (layer "F.Cu") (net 34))
 (segment (start 117.795 109.785) (end 116.62 110.96) (width 0.25) (layer "B.Cu") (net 34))
 (segment (start 117.795 96.635) (end 117.795 109.785) (width 0.25) (layer "B.Cu") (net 34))
 (segment (start 116.62 95.46) (end 117.795 96.635) (width 0.25) (layer "B.Cu") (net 34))
 (segment (start 114.08 108.42) (end 114.08 98) (width 0.25) (layer "F.Cu") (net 35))
 (segment (start 114.08 98) (end 114.08 108.42) (width 0.25) (layer "B.Cu") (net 35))
 (segment (start 115.255 109.785) (end 114.08 110.96) (width 0.25) (layer "F.Cu") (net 36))
 (segment (start 115.255 96.635) (end 115.255 109.785) (width 0.25) (layer "F.Cu") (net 36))
 (segment (start 114.08 95.46) (end 115.255 96.635) (width 0.25) (layer "F.Cu") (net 36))
 (segment (start 114.08 110.96) (end 115.255 109.785) (width 0.25) (layer "B.Cu") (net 36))
 (segment (start 115.255 96.635) (end 114.08 95.46) (width 0.25) (layer "B.Cu") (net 36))
 (segment (start 115.255 109.785) (end 115.255 96.635) (width 0.25) (layer "B.Cu") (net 36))
 (segment (start 111.54 98) (end 111.54 108.42) (width 0.25) (layer "F.Cu") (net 37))
 (segment (start 111.54 108.42) (end 111.54 98) (width 0.25) (layer "B.Cu") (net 37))
 (segment (start 112.715 96.635) (end 111.54 95.46) (width 0.25) (layer "F.Cu") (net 38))
 (segment (start 111.54 110.96) (end 112.715 109.785) (width 0.25) (layer "F.Cu") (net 38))
 (segment (start 112.715 109.785) (end 112.715 96.635) (width 0.25) (layer "F.Cu") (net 38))
 (segment (start 112.715 109.785) (end 111.54 110.96) (width 0.25) (layer "B.Cu") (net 38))
 (segment (start 112.715 96.635) (end 112.715 109.785) (width 0.25) (layer "B.Cu") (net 38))
 (segment (start 111.54 95.46) (end 112.715 96.635) (width 0.25) (layer "B.Cu") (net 38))
 (segment (start 109 98) (end 109 108.42) (width 0.25) (layer "F.Cu") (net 39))
 (segment (start 109 98) (end 109 108.42) (width 0.25) (layer "B.Cu") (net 39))
 (segment (start 109 95.46) (end 110.175 96.635) (width 0.25) (layer "F.Cu") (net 40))
 (segment (start 110.175 96.635) (end 110.175 109.785) (width 0.25) (layer "F.Cu") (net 40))
 (segment (start 110.175 109.785) (end 109 110.96) (width 0.25) (layer "F.Cu") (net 40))
 (segment (start 109 110.96) (end 110.175 109.785) (width 0.25) (layer "B.Cu") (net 40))
 (segment (start 110.175 109.785) (end 110.175 96.635) (width 0.25) (layer "B.Cu") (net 40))
 (segment (start 110.175 96.635) (end 109 95.46) (width 0.25) (layer "B.Cu") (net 40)))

